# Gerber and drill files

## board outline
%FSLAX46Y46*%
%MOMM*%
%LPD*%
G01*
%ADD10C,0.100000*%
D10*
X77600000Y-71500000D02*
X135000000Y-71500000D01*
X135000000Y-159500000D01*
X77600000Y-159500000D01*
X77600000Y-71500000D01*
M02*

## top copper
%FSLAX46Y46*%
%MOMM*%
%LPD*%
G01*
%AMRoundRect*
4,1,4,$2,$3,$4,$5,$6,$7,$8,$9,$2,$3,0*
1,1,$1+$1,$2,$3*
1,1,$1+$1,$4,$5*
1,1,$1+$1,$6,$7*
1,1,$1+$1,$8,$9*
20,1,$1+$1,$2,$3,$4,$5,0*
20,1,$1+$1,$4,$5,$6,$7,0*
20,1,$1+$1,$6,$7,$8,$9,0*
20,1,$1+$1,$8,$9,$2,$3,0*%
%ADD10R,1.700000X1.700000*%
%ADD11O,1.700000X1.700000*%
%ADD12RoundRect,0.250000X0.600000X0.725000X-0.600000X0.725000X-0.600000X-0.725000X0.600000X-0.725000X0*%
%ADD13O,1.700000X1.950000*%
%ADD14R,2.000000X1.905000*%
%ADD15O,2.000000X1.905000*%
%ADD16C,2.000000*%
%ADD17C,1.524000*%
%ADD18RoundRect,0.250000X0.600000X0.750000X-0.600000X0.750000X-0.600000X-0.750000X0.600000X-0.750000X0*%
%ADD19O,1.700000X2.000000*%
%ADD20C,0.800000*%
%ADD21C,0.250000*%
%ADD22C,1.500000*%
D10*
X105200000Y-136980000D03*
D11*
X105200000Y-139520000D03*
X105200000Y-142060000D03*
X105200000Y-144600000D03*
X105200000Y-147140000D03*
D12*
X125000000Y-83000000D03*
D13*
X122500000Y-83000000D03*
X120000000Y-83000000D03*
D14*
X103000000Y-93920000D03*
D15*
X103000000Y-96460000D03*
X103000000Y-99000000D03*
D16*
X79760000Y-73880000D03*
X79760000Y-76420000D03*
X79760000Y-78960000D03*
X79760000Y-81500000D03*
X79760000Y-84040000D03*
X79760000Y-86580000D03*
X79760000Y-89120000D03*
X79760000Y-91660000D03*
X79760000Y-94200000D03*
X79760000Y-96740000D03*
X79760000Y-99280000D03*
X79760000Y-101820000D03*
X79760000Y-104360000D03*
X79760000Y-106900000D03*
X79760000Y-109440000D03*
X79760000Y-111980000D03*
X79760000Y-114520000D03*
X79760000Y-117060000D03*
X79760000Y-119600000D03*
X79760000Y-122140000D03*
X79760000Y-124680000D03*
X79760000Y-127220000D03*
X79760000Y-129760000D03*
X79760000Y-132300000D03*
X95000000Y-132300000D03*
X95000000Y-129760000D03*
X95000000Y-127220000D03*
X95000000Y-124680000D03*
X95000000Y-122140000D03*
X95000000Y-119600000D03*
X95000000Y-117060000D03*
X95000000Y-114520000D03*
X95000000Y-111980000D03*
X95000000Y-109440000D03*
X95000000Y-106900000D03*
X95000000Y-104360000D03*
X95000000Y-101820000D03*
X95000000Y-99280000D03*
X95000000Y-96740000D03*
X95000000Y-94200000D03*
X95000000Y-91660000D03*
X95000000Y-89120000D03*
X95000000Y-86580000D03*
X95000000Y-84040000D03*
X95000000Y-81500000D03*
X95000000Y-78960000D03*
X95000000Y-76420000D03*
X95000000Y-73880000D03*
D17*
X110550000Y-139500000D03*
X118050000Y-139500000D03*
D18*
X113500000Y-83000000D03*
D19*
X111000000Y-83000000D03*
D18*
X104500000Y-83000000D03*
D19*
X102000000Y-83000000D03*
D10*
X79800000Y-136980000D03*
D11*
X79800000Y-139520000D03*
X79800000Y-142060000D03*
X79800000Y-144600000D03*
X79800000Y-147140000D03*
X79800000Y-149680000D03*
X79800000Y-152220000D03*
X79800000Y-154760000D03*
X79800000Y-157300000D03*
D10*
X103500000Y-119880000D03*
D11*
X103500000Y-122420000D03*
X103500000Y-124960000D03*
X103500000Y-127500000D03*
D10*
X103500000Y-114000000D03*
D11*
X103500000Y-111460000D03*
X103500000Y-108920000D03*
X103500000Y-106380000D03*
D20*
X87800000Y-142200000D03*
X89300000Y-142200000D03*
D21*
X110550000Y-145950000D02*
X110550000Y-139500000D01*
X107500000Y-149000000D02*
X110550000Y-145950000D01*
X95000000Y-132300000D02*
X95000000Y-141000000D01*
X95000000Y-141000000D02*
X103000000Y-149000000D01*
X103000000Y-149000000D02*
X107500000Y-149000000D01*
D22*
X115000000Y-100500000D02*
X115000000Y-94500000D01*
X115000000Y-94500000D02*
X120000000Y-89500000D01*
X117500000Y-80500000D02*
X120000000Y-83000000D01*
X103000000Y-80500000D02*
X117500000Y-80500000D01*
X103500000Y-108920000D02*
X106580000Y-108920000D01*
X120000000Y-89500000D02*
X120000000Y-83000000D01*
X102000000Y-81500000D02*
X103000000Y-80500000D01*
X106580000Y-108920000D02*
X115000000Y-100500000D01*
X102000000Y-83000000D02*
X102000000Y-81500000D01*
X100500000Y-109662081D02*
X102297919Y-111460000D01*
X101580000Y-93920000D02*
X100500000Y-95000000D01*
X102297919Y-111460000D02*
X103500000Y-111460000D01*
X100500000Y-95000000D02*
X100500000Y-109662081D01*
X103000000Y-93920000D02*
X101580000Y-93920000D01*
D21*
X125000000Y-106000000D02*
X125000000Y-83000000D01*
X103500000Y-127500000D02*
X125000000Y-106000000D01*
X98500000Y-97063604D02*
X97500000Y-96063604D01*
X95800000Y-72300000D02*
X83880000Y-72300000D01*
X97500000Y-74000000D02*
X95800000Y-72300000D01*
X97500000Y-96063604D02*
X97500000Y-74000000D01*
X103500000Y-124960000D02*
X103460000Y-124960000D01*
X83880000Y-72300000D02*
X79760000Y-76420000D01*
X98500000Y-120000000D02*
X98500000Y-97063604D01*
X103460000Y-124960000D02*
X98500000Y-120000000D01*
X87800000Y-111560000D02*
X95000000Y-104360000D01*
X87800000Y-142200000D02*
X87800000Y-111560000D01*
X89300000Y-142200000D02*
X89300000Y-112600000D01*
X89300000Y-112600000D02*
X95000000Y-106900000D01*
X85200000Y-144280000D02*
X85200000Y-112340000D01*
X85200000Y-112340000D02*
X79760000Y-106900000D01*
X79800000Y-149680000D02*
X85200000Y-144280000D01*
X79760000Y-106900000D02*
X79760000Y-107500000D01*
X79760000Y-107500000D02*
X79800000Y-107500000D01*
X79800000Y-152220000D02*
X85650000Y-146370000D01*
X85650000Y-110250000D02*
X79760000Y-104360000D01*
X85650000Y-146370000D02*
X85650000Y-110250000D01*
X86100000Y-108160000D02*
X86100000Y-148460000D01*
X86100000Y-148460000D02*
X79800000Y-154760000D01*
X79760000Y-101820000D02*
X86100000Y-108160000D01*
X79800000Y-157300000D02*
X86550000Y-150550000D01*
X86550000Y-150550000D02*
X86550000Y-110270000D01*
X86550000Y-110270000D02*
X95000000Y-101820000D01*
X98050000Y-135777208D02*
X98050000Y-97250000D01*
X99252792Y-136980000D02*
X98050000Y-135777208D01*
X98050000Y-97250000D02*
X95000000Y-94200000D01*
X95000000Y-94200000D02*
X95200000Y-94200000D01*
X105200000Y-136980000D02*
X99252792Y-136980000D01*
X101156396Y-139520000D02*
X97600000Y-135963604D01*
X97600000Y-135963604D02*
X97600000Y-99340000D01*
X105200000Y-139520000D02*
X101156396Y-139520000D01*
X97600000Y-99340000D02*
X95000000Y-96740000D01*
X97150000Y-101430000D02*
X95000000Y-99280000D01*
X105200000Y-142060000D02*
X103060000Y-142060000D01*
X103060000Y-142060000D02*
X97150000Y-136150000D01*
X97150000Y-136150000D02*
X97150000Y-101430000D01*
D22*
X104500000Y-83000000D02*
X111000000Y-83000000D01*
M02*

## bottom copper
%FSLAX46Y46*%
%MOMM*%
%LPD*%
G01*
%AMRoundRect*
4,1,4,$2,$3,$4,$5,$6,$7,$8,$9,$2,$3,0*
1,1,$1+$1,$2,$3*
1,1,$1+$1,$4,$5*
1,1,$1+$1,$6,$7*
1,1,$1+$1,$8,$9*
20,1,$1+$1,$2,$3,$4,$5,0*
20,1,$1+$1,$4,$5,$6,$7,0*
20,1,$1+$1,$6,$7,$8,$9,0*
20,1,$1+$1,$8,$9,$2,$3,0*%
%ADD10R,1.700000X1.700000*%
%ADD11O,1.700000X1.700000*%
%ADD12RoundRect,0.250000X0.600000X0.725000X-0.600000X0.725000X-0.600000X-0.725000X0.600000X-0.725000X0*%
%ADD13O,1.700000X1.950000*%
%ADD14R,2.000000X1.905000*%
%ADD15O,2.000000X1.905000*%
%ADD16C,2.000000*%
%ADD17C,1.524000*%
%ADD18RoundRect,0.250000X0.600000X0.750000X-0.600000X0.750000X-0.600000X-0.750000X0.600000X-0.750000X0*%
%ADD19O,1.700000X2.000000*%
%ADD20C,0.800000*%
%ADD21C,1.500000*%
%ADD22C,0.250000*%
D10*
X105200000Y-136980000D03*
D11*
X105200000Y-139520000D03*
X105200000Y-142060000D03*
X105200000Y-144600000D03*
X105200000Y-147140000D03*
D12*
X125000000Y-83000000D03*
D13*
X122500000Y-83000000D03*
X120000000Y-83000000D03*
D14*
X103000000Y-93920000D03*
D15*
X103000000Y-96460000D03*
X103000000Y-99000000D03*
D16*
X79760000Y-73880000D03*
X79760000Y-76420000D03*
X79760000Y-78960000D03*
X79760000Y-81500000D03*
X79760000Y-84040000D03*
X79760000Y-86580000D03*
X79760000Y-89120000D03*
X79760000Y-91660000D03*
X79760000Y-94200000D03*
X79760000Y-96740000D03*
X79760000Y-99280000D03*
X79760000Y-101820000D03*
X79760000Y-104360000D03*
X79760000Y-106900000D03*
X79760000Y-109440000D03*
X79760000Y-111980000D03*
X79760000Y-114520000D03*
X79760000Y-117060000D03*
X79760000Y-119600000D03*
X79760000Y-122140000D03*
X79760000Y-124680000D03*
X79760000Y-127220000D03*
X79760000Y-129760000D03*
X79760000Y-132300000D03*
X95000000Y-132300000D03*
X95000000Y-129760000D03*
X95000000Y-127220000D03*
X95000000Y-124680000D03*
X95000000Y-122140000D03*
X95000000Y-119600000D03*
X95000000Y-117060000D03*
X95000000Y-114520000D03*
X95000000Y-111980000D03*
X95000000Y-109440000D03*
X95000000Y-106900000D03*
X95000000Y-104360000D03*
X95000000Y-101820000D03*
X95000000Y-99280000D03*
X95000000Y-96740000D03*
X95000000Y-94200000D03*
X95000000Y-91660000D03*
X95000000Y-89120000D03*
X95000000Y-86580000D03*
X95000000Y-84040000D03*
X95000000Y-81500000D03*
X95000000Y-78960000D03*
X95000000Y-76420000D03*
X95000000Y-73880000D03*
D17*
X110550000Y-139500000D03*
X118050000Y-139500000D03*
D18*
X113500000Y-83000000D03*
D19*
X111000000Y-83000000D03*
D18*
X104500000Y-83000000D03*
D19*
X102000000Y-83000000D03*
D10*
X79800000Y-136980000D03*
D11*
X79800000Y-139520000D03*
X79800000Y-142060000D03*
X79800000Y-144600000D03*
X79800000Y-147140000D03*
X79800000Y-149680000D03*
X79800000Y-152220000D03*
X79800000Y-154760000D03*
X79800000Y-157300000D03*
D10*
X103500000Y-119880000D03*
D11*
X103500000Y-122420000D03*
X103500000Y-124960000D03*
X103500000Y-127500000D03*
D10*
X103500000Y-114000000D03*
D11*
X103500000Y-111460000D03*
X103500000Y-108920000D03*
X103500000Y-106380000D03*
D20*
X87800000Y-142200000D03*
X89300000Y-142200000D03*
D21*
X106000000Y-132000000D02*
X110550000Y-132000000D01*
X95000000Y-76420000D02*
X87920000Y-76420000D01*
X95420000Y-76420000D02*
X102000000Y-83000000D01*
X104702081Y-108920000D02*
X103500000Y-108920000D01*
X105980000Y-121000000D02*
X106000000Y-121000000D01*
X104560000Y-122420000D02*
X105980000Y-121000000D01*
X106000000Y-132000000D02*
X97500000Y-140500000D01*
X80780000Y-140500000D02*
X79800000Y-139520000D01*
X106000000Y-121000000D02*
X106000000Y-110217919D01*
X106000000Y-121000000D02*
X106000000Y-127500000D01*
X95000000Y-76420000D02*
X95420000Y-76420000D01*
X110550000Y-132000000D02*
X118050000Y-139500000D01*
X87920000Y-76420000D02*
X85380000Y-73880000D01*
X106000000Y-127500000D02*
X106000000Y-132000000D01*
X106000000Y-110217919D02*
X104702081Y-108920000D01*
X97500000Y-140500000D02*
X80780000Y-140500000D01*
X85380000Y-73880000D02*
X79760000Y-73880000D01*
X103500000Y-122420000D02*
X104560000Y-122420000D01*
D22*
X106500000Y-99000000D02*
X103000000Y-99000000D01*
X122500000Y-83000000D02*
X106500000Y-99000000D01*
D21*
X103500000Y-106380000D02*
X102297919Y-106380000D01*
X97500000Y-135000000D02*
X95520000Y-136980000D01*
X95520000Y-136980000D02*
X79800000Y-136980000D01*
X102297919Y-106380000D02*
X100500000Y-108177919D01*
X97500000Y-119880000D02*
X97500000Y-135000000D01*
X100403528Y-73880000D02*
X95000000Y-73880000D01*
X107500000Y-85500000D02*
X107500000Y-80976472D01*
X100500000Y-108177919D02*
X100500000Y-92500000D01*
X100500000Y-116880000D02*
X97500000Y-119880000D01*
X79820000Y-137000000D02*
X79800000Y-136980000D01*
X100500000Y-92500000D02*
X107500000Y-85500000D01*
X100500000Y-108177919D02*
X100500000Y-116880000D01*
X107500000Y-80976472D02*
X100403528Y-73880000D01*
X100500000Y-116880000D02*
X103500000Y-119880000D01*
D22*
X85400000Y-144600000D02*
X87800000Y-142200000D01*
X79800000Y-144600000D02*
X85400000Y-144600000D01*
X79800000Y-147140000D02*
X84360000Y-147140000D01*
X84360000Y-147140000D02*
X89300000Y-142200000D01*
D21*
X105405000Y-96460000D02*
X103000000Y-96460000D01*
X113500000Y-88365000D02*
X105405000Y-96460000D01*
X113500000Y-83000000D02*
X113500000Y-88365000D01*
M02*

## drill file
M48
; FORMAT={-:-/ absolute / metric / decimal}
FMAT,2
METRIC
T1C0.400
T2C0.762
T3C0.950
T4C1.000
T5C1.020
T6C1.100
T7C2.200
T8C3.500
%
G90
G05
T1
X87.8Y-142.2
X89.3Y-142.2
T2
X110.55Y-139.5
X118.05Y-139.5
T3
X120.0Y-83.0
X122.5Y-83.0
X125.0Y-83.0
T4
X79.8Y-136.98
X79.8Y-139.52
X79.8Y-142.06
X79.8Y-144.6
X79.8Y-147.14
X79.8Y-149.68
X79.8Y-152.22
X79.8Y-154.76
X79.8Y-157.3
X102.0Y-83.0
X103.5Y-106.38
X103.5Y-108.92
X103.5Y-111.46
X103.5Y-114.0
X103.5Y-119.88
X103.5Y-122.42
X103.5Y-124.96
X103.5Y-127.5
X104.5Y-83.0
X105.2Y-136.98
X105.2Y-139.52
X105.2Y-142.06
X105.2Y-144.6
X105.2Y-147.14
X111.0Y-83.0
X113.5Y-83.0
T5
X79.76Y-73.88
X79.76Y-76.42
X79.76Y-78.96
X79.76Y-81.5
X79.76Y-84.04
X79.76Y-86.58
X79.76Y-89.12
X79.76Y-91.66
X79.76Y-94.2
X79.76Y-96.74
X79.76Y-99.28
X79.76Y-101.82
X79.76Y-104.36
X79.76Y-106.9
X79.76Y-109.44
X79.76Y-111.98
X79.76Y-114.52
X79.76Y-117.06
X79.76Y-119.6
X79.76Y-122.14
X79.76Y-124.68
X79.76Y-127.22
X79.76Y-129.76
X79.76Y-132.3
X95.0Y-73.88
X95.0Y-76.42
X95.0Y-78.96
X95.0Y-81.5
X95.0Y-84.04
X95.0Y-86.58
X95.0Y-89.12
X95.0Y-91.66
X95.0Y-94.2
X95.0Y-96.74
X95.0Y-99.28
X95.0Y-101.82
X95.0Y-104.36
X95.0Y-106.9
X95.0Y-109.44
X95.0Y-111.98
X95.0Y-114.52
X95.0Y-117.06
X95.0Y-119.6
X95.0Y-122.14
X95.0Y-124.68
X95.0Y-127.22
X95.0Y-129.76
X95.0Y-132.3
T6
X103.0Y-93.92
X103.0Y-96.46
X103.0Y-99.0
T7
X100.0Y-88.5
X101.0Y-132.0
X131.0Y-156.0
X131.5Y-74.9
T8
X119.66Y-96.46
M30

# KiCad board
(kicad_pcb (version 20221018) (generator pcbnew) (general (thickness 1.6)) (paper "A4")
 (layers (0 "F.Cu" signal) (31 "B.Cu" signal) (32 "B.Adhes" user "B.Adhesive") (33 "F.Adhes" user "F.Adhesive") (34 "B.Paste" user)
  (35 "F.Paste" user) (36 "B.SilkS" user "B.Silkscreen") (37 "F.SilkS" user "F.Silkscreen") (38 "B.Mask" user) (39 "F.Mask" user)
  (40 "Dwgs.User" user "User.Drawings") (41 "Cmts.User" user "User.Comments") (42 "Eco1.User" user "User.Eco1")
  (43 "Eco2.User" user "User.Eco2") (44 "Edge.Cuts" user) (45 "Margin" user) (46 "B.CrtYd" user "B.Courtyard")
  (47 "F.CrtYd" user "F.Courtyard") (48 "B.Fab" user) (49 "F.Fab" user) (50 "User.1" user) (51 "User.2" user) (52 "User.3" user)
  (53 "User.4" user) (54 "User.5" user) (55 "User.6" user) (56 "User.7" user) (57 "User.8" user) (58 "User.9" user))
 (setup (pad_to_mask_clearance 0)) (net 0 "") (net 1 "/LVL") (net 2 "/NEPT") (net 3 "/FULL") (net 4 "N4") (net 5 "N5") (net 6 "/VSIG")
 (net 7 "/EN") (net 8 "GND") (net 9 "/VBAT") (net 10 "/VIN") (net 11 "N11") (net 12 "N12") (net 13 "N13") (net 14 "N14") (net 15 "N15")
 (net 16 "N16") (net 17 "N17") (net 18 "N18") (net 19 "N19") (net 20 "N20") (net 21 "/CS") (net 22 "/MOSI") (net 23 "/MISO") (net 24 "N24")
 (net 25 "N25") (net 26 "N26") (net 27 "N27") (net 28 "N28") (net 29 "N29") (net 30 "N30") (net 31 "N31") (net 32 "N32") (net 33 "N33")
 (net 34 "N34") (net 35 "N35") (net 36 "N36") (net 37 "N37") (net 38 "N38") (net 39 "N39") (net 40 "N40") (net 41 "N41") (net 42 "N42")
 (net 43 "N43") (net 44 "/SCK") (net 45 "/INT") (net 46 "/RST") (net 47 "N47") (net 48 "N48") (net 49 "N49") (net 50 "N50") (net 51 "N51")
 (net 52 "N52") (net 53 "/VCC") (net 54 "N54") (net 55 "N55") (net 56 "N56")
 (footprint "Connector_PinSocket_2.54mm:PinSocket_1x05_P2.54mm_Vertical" (layer "F.Cu") (at 105.2 136.98)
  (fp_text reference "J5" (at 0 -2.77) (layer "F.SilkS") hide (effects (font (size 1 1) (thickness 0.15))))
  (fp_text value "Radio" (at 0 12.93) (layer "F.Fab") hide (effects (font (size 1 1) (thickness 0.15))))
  (pad "1" thru_hole rect (at 0 0) (size 1.7 1.7) (drill 1) (layers "*.Cu" "*.Mask") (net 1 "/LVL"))
  (pad "2" thru_hole oval (at 0 2.54) (size 1.7 1.7) (drill 1) (layers "*.Cu" "*.Mask") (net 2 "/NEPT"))
  (pad "3" thru_hole oval (at 0 5.08) (size 1.7 1.7) (drill 1) (layers "*.Cu" "*.Mask") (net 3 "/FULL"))
  (pad "4" thru_hole oval (at 0 7.62) (size 1.7 1.7) (drill 1) (layers "*.Cu" "*.Mask") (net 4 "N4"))
  (pad "5" thru_hole oval (at 0 10.16) (size 1.7 1.7) (drill 1) (layers "*.Cu" "*.Mask") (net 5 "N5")))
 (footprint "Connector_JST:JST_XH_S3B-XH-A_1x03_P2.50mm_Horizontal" (layer "F.Cu") (at 125 83 180)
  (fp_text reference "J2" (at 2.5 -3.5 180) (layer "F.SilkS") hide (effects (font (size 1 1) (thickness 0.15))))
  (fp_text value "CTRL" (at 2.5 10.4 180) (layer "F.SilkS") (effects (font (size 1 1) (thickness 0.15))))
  (pad "1" thru_hole roundrect (at 0 0 180) (size 1.7 1.95) (drill 0.95) (layers "*.Cu" "*.Mask") (roundrect_rratio 0.1470588235)
   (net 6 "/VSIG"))
  (pad "2" thru_hole oval (at 2.5 0 180) (size 1.7 1.95) (drill 0.95) (layers "*.Cu" "*.Mask") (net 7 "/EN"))
  (pad "3" thru_hole oval (at 5 0 180) (size 1.7 1.95) (drill 0.95) (layers "*.Cu" "*.Mask") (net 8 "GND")))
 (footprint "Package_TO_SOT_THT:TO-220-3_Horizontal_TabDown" (layer "F.Cu") (at 103 93.92 -90)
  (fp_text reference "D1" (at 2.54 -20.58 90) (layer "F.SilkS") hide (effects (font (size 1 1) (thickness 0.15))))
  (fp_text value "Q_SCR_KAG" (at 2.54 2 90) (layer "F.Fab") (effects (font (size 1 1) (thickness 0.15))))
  (pad "" np_thru_hole oval (at 2.54 -16.66 270) (size 3.5 3.5) (drill 3.5) (layers "*.Cu" "*.Mask"))
  (pad "1" thru_hole rect (at 0 0 270) (size 1.905 2) (drill 1.1) (layers "*.Cu" "*.Mask") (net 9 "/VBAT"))
  (pad "2" thru_hole oval (at 2.54 0 270) (size 1.905 2) (drill 1.1) (layers "*.Cu" "*.Mask") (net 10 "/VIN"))
  (pad "3" thru_hole oval (at 5.08 0 270) (size 1.905 2) (drill 1.1) (layers "*.Cu" "*.Mask") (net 7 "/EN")))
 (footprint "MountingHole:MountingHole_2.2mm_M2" (layer "F.Cu") (at 131 156)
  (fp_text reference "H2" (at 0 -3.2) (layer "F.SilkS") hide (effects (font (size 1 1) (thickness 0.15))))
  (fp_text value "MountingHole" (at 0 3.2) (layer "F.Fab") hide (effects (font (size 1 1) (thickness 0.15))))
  (pad "" np_thru_hole circle (at 0 0) (size 2.2 2.2) (drill 2.2) (layers "*.Cu" "*.Mask")))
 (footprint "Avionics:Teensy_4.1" (layer "F.Cu") (at 87.38 103.09)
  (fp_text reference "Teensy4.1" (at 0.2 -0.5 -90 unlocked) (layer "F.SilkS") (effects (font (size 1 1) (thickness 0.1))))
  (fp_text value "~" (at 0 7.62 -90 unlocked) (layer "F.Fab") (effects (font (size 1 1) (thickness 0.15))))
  (pad "0" thru_hole circle (at -7.62 -29.21) (size 2 2) (drill 1.02) (layers "*.Cu" "*.Mask") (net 8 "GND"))
  (pad "1" thru_hole circle (at -7.62 -26.67) (size 2 2) (drill 1.02) (layers "*.Cu" "*.Mask") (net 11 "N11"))
  (pad "2" thru_hole circle (at -7.62 -24.13) (size 2 2) (drill 1.02) (layers "*.Cu" "*.Mask") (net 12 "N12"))
  (pad "3" thru_hole circle (at -7.62 -21.59) (size 2 2) (drill 1.02) (layers "*.Cu" "*.Mask") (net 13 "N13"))
  (pad "4" thru_hole circle (at -7.62 -19.05) (size 2 2) (drill 1.02) (layers "*.Cu" "*.Mask") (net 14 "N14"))
  (pad "5" thru_hole circle (at -7.62 -16.51) (size 2 2) (drill 1.02) (layers "*.Cu" "*.Mask") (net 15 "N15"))
  (pad "6" thru_hole circle (at -7.62 -13.97) (size 2 2) (drill 1.02) (layers "*.Cu" "*.Mask") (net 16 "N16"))
  (pad "7" thru_hole circle (at -7.62 -11.43) (size 2 2) (drill 1.02) (layers "*.Cu" "*.Mask") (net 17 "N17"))
  (pad "8" thru_hole circle (at -7.62 -8.89) (size 2 2) (drill 1.02) (layers "*.Cu" "*.Mask") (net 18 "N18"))
  (pad "9" thru_hole circle (at -7.62 -6.35) (size 2 2) (drill 1.02) (layers "*.Cu" "*.Mask") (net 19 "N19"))
  (pad "10" thru_hole circle (at -7.62 -3.81) (size 2 2) (drill 1.02) (layers "*.Cu" "*.Mask") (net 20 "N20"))
  (pad "11" thru_hole circle (at -7.62 -1.27) (size 2 2) (drill 1.02) (layers "*.Cu" "*.Mask") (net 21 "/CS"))
  (pad "12" thru_hole circle (at -7.62 1.27) (size 2 2) (drill 1.02) (layers "*.Cu" "*.Mask") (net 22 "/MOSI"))
  (pad "13" thru_hole circle (at -7.62 3.81) (size 2 2) (drill 1.02) (layers "*.Cu" "*.Mask") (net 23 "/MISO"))
  (pad "14" thru_hole circle (at -7.62 6.35) (size 2 2) (drill 1.02) (layers "*.Cu" "*.Mask") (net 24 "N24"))
  (pad "15" thru_hole circle (at -7.62 8.89) (size 2 2) (drill 1.02) (layers "*.Cu" "*.Mask") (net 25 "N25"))
  (pad "16" thru_hole circle (at -7.62 11.43) (size 2 2) (drill 1.02) (layers "*.Cu" "*.Mask") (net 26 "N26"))
  (pad "17" thru_hole circle (at -7.62 13.97) (size 2 2) (drill 1.02) (layers "*.Cu" "*.Mask") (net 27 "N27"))
  (pad "18" thru_hole circle (at -7.62 16.51) (size 2 2) (drill 1.02) (layers "*.Cu" "*.Mask") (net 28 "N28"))
  (pad "19" thru_hole circle (at -7.62 19.05) (size 2 2) (drill 1.02) (layers "*.Cu" "*.Mask") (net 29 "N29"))
  (pad "20" thru_hole circle (at -7.62 21.59) (size 2 2) (drill 1.02) (layers "*.Cu" "*.Mask") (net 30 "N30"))
  (pad "21" thru_hole circle (at -7.62 24.13) (size 2 2) (drill 1.02) (layers "*.Cu" "*.Mask") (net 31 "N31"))
  (pad "22" thru_hole circle (at -7.62 26.67) (size 2 2) (drill 1.02) (layers "*.Cu" "*.Mask") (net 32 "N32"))
  (pad "23" thru_hole circle (at -7.62 29.21) (size 2 2) (drill 1.02) (layers "*.Cu" "*.Mask") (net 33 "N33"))
  (pad "24" thru_hole circle (at 7.62 29.21) (size 2 2) (drill 1.02) (layers "*.Cu" "*.Mask") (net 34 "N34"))
  (pad "25" thru_hole circle (at 7.62 26.67) (size 2 2) (drill 1.02) (layers "*.Cu" "*.Mask") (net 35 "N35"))
  (pad "26" thru_hole circle (at 7.62 24.13) (size 2 2) (drill 1.02) (layers "*.Cu" "*.Mask") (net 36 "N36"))
  (pad "27" thru_hole circle (at 7.62 21.59) (size 2 2) (drill 1.02) (layers "*.Cu" "*.Mask") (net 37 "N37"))
  (pad "28" thru_hole circle (at 7.62 19.05) (size 2 2) (drill 1.02) (layers "*.Cu" "*.Mask") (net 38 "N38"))
  (pad "29" thru_hole circle (at 7.62 16.51) (size 2 2) (drill 1.02) (layers "*.Cu" "*.Mask") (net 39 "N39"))
  (pad "30" thru_hole circle (at 7.62 13.97) (size 2 2) (drill 1.02) (layers "*.Cu" "*.Mask") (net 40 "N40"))
  (pad "31" thru_hole circle (at 7.62 11.43) (size 2 2) (drill 1.02) (layers "*.Cu" "*.Mask") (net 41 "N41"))
  (pad "32" thru_hole circle (at 7.62 8.89) (size 2 2) (drill 1.02) (layers "*.Cu" "*.Mask") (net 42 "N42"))
  (pad "33" thru_hole circle (at 7.62 6.35) (size 2 2) (drill 1.02) (layers "*.Cu" "*.Mask") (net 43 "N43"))
  (pad "34" thru_hole circle (at 7.62 3.81) (size 2 2) (drill 1.02) (layers "*.Cu" "*.Mask") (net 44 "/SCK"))
  (pad "35" thru_hole circle (at 7.62 1.27) (size 2 2) (drill 1.02) (layers "*.Cu" "*.Mask") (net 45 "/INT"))
  (pad "36" thru_hole circle (at 7.62 -1.27) (size 2 2) (drill 1.02) (layers "*.Cu" "*.Mask") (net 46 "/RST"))
  (pad "37" thru_hole circle (at 7.62 -3.81) (size 2 2) (drill 1.02) (layers "*.Cu" "*.Mask") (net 3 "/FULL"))
  (pad "38" thru_hole circle (at 7.62 -6.35) (size 2 2) (drill 1.02) (layers "*.Cu" "*.Mask") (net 2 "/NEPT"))
  (pad "39" thru_hole circle (at 7.62 -8.89) (size 2 2) (drill 1.02) (layers "*.Cu" "*.Mask") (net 1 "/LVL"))
  (pad "40" thru_hole circle (at 7.62 -11.43) (size 2 2) (drill 1.02) (layers "*.Cu" "*.Mask") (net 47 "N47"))
  (pad "41" thru_hole circle (at 7.62 -13.97) (size 2 2) (drill 1.02) (layers "*.Cu" "*.Mask") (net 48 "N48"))
  (pad "42" thru_hole circle (at 7.62 -16.51) (size 2 2) (drill 1.02) (layers "*.Cu" "*.Mask") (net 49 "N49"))
  (pad "43" thru_hole circle (at 7.62 -19.05) (size 2 2) (drill 1.02) (layers "*.Cu" "*.Mask") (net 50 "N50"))
  (pad "44" thru_hole circle (at 7.62 -21.59) (size 2 2) (drill 1.02) (layers "*.Cu" "*.Mask") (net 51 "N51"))
  (pad "45" thru_hole circle (at 7.62 -24.13) (size 2 2) (drill 1.02) (layers "*.Cu" "*.Mask") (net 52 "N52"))
  (pad "46" thru_hole circle (at 7.62 -26.67) (size 2 2) (drill 1.02) (layers "*.Cu" "*.Mask") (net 8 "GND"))
  (pad "47" thru_hole circle (at 7.62 -29.21) (size 2 2) (drill 1.02) (layers "*.Cu" "*.Mask") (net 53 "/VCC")))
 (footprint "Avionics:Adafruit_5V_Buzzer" (layer "F.Cu") (at 114.3 144)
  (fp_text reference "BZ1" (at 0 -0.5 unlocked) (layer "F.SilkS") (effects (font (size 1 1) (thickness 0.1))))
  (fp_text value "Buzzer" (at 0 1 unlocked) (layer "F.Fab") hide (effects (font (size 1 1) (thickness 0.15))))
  (pad "1" thru_hole circle (at -3.75 -4.5) (size 1.524 1.524) (drill 0.762) (layers "*.Cu" "*.Mask") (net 34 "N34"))
  (pad "2" thru_hole circle (at 3.75 -4.5) (size 1.524 1.524) (drill 0.762) (layers "*.Cu" "*.Mask") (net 8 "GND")))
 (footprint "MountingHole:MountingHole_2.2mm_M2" (layer "F.Cu") (at 131.5 74.9)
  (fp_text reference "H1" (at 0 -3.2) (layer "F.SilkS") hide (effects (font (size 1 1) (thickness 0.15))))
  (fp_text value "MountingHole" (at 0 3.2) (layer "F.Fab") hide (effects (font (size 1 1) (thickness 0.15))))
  (pad "" np_thru_hole circle (at 0 0) (size 2.2 2.2) (drill 2.2) (layers "*.Cu" "*.Mask")))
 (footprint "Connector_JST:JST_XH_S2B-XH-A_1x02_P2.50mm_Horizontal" (layer "F.Cu") (at 113.5 83 180)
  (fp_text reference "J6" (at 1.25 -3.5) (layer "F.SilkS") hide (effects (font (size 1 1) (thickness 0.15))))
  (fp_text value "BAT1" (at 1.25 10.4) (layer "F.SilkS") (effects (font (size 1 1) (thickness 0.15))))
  (pad "1" thru_hole roundrect (at 0 0 180) (size 1.7 2) (drill 1) (layers "*.Cu" "*.Mask") (roundrect_rratio 0.1470588235) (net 10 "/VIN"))
  (pad "2" thru_hole oval (at 2.5 0 180) (size 1.7 2) (drill 1) (layers "*.Cu" "*.Mask") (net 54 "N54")))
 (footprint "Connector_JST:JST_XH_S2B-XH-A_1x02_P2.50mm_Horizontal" (layer "F.Cu") (at 104.5 83 180)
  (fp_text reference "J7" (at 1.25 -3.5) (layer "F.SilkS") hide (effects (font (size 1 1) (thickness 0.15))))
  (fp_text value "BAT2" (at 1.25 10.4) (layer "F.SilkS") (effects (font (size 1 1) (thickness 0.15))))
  (pad "1" thru_hole roundrect (at 0 0 180) (size 1.7 2) (drill 1) (layers "*.Cu" "*.Mask") (roundrect_rratio 0.1470588235) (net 54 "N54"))
  (pad "2" thru_hole oval (at 2.5 0 180) (size 1.7 2) (drill 1) (layers "*.Cu" "*.Mask") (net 8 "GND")))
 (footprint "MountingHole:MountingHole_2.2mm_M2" (layer "F.Cu") (at 100 88.5)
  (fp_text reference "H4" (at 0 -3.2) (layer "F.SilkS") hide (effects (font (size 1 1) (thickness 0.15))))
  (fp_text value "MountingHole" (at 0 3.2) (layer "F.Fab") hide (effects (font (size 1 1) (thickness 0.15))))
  (pad "" np_thru_hole circle (at 0 0) (size 2.2 2.2) (drill 2.2) (layers "*.Cu" "*.Mask")))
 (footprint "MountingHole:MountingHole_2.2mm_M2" (layer "F.Cu") (at 101 132)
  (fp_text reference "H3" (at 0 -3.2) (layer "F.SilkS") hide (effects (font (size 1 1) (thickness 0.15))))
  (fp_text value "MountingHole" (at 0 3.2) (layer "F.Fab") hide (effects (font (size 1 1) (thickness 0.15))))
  (pad "" np_thru_hole circle (at 0 0) (size 2.2 2.2) (drill 2.2) (layers "*.Cu" "*.Mask")))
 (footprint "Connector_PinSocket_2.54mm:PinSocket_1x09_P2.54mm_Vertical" (layer "F.Cu") (at 79.8 136.98)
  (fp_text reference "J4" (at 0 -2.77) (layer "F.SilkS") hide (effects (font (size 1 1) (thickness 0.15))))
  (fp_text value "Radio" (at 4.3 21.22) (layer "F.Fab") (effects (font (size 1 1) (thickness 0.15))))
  (pad "1" thru_hole rect (at 0 0) (size 1.7 1.7) (drill 1) (layers "*.Cu" "*.Mask") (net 53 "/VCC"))
  (pad "2" thru_hole oval (at 0 2.54) (size 1.7 1.7) (drill 1) (layers "*.Cu" "*.Mask") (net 8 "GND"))
  (pad "3" thru_hole oval (at 0 5.08) (size 1.7 1.7) (drill 1) (layers "*.Cu" "*.Mask") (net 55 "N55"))
  (pad "4" thru_hole oval (at 0 7.62) (size 1.7 1.7) (drill 1) (layers "*.Cu" "*.Mask") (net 45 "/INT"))
  (pad "5" thru_hole oval (at 0 10.16) (size 1.7 1.7) (drill 1) (layers "*.Cu" "*.Mask") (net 44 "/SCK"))
  (pad "6" thru_hole oval (at 0 12.7) (size 1.7 1.7) (drill 1) (layers "*.Cu" "*.Mask") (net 23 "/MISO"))
  (pad "7" thru_hole oval (at 0 15.24) (size 1.7 1.7) (drill 1) (layers "*.Cu" "*.Mask") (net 22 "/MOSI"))
  (pad "8" thru_hole oval (at 0 17.78) (size 1.7 1.7) (drill 1) (layers "*.Cu" "*.Mask") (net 21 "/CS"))
  (pad "9" thru_hole oval (at 0 20.32) (size 1.7 1.7) (drill 1) (layers "*.Cu" "*.Mask") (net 46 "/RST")))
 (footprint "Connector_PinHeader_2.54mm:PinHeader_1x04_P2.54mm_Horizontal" (layer "F.Cu") (at 103.5 119.88)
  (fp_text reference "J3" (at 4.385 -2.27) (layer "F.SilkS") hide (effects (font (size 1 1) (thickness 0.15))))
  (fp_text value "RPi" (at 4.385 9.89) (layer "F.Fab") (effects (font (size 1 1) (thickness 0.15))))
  (pad "1" thru_hole rect (at 0 0) (size 1.7 1.7) (drill 1) (layers "*.Cu" "*.Mask") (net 53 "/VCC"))
  (pad "2" thru_hole oval (at 0 2.54) (size 1.7 1.7) (drill 1) (layers "*.Cu" "*.Mask") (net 8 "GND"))
  (pad "3" thru_hole oval (at 0 5.08) (size 1.7 1.7) (drill 1) (layers "*.Cu" "*.Mask") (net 11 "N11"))
  (pad "4" thru_hole oval (at 0 7.62) (size 1.7 1.7) (drill 1) (layers "*.Cu" "*.Mask") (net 6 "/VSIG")))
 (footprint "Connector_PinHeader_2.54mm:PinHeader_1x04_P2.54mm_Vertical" (layer "F.Cu") (at 103.5 114 180)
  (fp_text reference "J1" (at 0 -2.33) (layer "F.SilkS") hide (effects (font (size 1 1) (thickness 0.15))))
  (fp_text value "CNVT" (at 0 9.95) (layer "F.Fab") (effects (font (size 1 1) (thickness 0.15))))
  (pad "1" thru_hole rect (at 0 0 180) (size 1.7 1.7) (drill 1) (layers "*.Cu" "*.Mask") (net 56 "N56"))
  (pad "2" thru_hole oval (at 0 2.54 180) (size 1.7 1.7) (drill 1) (layers "*.Cu" "*.Mask") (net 9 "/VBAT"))
  (pad "3" thru_hole oval (at 0 5.08 180) (size 1.7 1.7) (drill 1) (layers "*.Cu" "*.Mask") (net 8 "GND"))
  (pad "4" thru_hole oval (at 0 7.62 180) (size 1.7 1.7) (drill 1) (layers "*.Cu" "*.Mask") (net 53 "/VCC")))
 (gr_rect (start 77.6 71.5) (end 135 159.5) (stroke (width 0.1) (type default)) (fill none) (layer "Edge.Cuts"))
 (segment (start 110.55 145.95) (end 110.55 139.5) (width 0.25) (layer "F.Cu") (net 34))
 (segment (start 107.5 149) (end 110.55 145.95) (width 0.25) (layer "F.Cu") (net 34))
 (segment (start 95 132.3) (end 95 141) (width 0.25) (layer "F.Cu") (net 34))
 (segment (start 95 141) (end 103 149) (width 0.25) (layer "F.Cu") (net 34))
 (segment (start 103 149) (end 107.5 149) (width 0.25) (layer "F.Cu") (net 34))
 (segment (start 115 100.5) (end 115 94.5) (width 1.5) (layer "F.Cu") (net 8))
 (segment (start 115 94.5) (end 120 89.5) (width 1.5) (layer "F.Cu") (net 8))
 (segment (start 117.5 80.5) (end 120 83) (width 1.5) (layer "F.Cu") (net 8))
 (segment (start 103 80.5) (end 117.5 80.5) (width 1.5) (layer "F.Cu") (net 8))
 (segment (start 103.5 108.92) (end 106.58 108.92) (width 1.5) (layer "F.Cu") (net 8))
 (segment (start 120 89.5) (end 120 83) (width 1.5) (layer "F.Cu") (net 8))
 (segment (start 102 81.5) (end 103 80.5) (width 1.5) (layer "F.Cu") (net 8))
 (segment (start 106.58 108.92) (end 115 100.5) (width 1.5) (layer "F.Cu") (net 8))
 (segment (start 102 83) (end 102 81.5) (width 1.5) (layer "F.Cu") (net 8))
 (segment (start 106 132) (end 110.55 132) (width 1.5) (layer "B.Cu") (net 8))
 (segment (start 95 76.42) (end 87.92 76.42) (width 1.5) (layer "B.Cu") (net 8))
 (segment (start 95.42 76.42) (end 102 83) (width 1.5) (layer "B.Cu") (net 8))
 (segment (start 104.702081 108.92) (end 103.5 108.92) (width 1.5) (layer "B.Cu") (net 8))
 (segment (start 105.98 121) (end 106 121) (width 1.5) (layer "B.Cu") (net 8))
 (segment (start 104.56 122.42) (end 105.98 121) (width 1.5) (layer "B.Cu") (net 8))
 (segment (start 106 132) (end 97.5 140.5) (width 1.5) (layer "B.Cu") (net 8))
 (segment (start 80.78 140.5) (end 79.8 139.52) (width 1.5) (layer "B.Cu") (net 8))
 (segment (start 106 121) (end 106 110.217919) (width 1.5) (layer "B.Cu") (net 8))
 (segment (start 106 121) (end 106 127.5) (width 1.5) (layer "B.Cu") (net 8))
 (segment (start 95 76.42) (end 95.42 76.42) (width 1.5) (layer "B.Cu") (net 8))
 (segment (start 110.55 132) (end 118.05 139.5) (width 1.5) (layer "B.Cu") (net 8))
 (segment (start 87.92 76.42) (end 85.38 73.88) (width 1.5) (layer "B.Cu") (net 8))
 (segment (start 106 127.5) (end 106 132) (width 1.5) (layer "B.Cu") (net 8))
 (segment (start 106 110.217919) (end 104.702081 108.92) (width 1.5) (layer "B.Cu") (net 8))
 (segment (start 97.5 140.5) (end 80.78 140.5) (width 1.5) (layer "B.Cu") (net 8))
 (segment (start 85.38 73.88) (end 79.76 73.88) (width 1.5) (layer "B.Cu") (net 8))
 (segment (start 103.5 122.42) (end 104.56 122.42) (width 1.5) (layer "B.Cu") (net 8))
 (segment (start 106.5 99) (end 103 99) (width 0.25) (layer "B.Cu") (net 7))
 (segment (start 122.5 83) (end 106.5 99) (width 0.25) (layer "B.Cu") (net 7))
 (segment (start 100.5 109.662081) (end 102.297919 111.46) (width 1.5) (layer "F.Cu") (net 9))
 (segment (start 101.58 93.92) (end 100.5 95) (width 1.5) (layer "F.Cu") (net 9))
 (segment (start 102.297919 111.46) (end 103.5 111.46) (width 1.5) (layer "F.Cu") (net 9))
 (segment (start 100.5 95) (end 100.5 109.662081) (width 1.5) (layer "F.Cu") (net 9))
 (segment (start 103 93.92) (end 101.58 93.92) (width 1.5) (layer "F.Cu") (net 9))
 (segment (start 103.5 106.38) (end 102.297919 106.38) (width 1.5) (layer "B.Cu") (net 53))
 (segment (start 97.5 135) (end 95.52 136.98) (width 1.5) (layer "B.Cu") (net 53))
 (segment (start 95.52 136.98) (end 79.8 136.98) (width 1.5) (layer "B.Cu") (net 53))
 (segment (start 102.297919 106.38) (end 100.5 108.177919) (width 1.5) (layer "B.Cu") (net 53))
 (segment (start 97.5 119.88) (end 97.5 135) (width 1.5) (layer "B.Cu") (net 53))
 (segment (start 100.403528 73.88) (end 95 73.88) (width 1.5) (layer "B.Cu") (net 53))
 (segment (start 107.5 85.5) (end 107.5 80.976472) (width 1.5) (layer "B.Cu") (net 53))
 (segment (start 100.5 108.177919) (end 100.5 92.5) (width 1.5) (layer "B.Cu") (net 53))
 (segment (start 100.5 116.88) (end 97.5 119.88) (width 1.5) (layer "B.Cu") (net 53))
 (segment (start 79.82 137) (end 79.8 136.98) (width 1.5) (layer "B.Cu") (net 53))
 (segment (start 100.5 92.5) (end 107.5 85.5) (width 1.5) (layer "B.Cu") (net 53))
 (segment (start 100.5 108.177919) (end 100.5 116.88) (width 1.5) (layer "B.Cu") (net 53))
 (segment (start 107.5 80.976472) (end 100.403528 73.88) (width 1.5) (layer "B.Cu") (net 53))
 (segment (start 100.5 116.88) (end 103.5 119.88) (width 1.5) (layer "B.Cu") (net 53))
 (segment (start 125 106) (end 125 83) (width 0.25) (layer "F.Cu") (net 6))
 (segment (start 103.5 127.5) (end 125 106) (width 0.25) (layer "F.Cu") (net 6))
 (segment (start 98.5 97.063604) (end 97.5 96.063604) (width 0.25) (layer "F.Cu") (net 11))
 (segment (start 95.8 72.3) (end 83.88 72.3) (width 0.25) (layer "F.Cu") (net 11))
 (segment (start 97.5 74) (end 95.8 72.3) (width 0.25) (layer "F.Cu") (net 11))
 (segment (start 97.5 96.063604) (end 97.5 74) (width 0.25) (layer "F.Cu") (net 11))
 (segment (start 103.5 124.96) (end 103.46 124.96) (width 0.25) (layer "F.Cu") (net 11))
 (segment (start 83.88 72.3) (end 79.76 76.42) (width 0.25) (layer "F.Cu") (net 11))
 (segment (start 98.5 120) (end 98.5 97.063604) (width 0.25) (layer "F.Cu") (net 11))
 (segment (start 103.46 124.96) (end 98.5 120) (width 0.25) (layer "F.Cu") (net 11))
 (segment (start 87.8 111.56) (end 95 104.36) (width 0.25) (layer "F.Cu") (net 45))
 (segment (start 87.8 142.2) (end 87.8 111.56) (width 0.25) (layer "F.Cu") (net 45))
 (via (at 87.8 142.2) (size 0.8) (drill 0.4) (layers "F.Cu" "B.Cu") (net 45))
 (segment (start 85.4 144.6) (end 87.8 142.2) (width 0.25) (layer "B.Cu") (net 45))
 (segment (start 79.8 144.6) (end 85.4 144.6) (width 0.25) (layer "B.Cu") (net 45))
 (segment (start 89.3 142.2) (end 89.3 112.6) (width 0.25) (layer "F.Cu") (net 44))
 (segment (start 89.3 112.6) (end 95 106.9) (width 0.25) (layer "F.Cu") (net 44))
 (via (at 89.3 142.2) (size 0.8) (drill 0.4) (layers "F.Cu" "B.Cu") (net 44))
 (segment (start 79.8 147.14) (end 84.36 147.14) (width 0.25) (layer "B.Cu") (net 44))
 (segment (start 84.36 147.14) (end 89.3 142.2) (width 0.25) (layer "B.Cu") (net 44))
 (segment (start 85.2 144.28) (end 85.2 112.34) (width 0.25) (layer "F.Cu") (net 23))
 (segment (start 85.2 112.34) (end 79.76 106.9) (width 0.25) (layer "F.Cu") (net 23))
 (segment (start 79.8 149.68) (end 85.2 144.28) (width 0.25) (layer "F.Cu") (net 23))
 (segment (start 79.76 106.9) (end 79.76 107.5) (width 0.25) (layer "F.Cu") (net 23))
 (segment (start 79.76 107.5) (end 79.8 107.5) (width 0.25) (layer "F.Cu") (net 23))
 (segment (start 79.8 152.22) (end 85.65 146.37) (width 0.25) (layer "F.Cu") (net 22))
 (segment (start 85.65 110.25) (end 79.76 104.36) (width 0.25) (layer "F.Cu") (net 22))
 (segment (start 85.65 146.37) (end 85.65 110.25) (width 0.25) (layer "F.Cu") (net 22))
 (segment (start 86.1 108.16) (end 86.1 148.46) (width 0.25) (layer "F.Cu") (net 21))
 (segment (start 86.1 148.46) (end 79.8 154.76) (width 0.25) (layer "F.Cu") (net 21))
 (segment (start 79.76 101.82) (end 86.1 108.16) (width 0.25) (layer "F.Cu") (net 21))
 (segment (start 79.8 157.3) (end 86.55 150.55) (width 0.25) (layer "F.Cu") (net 46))
 (segment (start 86.55 150.55) (end 86.55 110.27) (width 0.25) (layer "F.Cu") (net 46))
 (segment (start 86.55 110.27) (end 95 101.82) (width 0.25) (layer "F.Cu") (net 46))
 (segment (start 98.05 135.777208) (end 98.05 97.25) (width 0.25) (layer "F.Cu") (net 1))
 (segment (start 99.252792 136.98) (end 98.05 135.777208) (width 0.25) (layer "F.Cu") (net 1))
 (segment (start 98.05 97.25) (end 95 94.2) (width 0.25) (layer "F.Cu") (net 1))
 (segment (start 95 94.2) (end 95.2 94.2) (width 0.25) (layer "F.Cu") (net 1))
 (segment (start 105.2 136.98) (end 99.252792 136.98) (width 0.25) (layer "F.Cu") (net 1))
 (segment (start 101.156396 139.52) (end 97.6 135.963604) (width 0.25) (layer "F.Cu") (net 2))
 (segment (start 97.6 135.963604) (end 97.6 99.34) (width 0.25) (layer "F.Cu") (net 2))
 (segment (start 105.2 139.52) (end 101.156396 139.52) (width 0.25) (layer "F.Cu") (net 2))
 (segment (start 97.6 99.34) (end 95 96.74) (width 0.25) (layer "F.Cu") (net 2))
 (segment (start 97.15 101.43) (end 95 99.28) (width 0.25) (layer "F.Cu") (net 3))
 (segment (start 105.2 142.06) (end 103.06 142.06) (width 0.25) (layer "F.Cu") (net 3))
 (segment (start 103.06 142.06) (end 97.15 136.15) (width 0.25) (layer "F.Cu") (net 3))
 (segment (start 97.15 136.15) (end 97.15 101.43) (width 0.25) (layer "F.Cu") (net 3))
 (segment (start 104.5 83) (end 111 83) (width 1.5) (layer "F.Cu") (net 54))
 (segment (start 105.405 96.46) (end 103 96.46) (width 1.5) (layer "B.Cu") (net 10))
 (segment (start 113.5 88.365) (end 105.405 96.46) (width 1.5) (layer "B.Cu") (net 10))
 (segment (start 113.5 83) (end 113.5 88.365) (width 1.5) (layer "B.Cu") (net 10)))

